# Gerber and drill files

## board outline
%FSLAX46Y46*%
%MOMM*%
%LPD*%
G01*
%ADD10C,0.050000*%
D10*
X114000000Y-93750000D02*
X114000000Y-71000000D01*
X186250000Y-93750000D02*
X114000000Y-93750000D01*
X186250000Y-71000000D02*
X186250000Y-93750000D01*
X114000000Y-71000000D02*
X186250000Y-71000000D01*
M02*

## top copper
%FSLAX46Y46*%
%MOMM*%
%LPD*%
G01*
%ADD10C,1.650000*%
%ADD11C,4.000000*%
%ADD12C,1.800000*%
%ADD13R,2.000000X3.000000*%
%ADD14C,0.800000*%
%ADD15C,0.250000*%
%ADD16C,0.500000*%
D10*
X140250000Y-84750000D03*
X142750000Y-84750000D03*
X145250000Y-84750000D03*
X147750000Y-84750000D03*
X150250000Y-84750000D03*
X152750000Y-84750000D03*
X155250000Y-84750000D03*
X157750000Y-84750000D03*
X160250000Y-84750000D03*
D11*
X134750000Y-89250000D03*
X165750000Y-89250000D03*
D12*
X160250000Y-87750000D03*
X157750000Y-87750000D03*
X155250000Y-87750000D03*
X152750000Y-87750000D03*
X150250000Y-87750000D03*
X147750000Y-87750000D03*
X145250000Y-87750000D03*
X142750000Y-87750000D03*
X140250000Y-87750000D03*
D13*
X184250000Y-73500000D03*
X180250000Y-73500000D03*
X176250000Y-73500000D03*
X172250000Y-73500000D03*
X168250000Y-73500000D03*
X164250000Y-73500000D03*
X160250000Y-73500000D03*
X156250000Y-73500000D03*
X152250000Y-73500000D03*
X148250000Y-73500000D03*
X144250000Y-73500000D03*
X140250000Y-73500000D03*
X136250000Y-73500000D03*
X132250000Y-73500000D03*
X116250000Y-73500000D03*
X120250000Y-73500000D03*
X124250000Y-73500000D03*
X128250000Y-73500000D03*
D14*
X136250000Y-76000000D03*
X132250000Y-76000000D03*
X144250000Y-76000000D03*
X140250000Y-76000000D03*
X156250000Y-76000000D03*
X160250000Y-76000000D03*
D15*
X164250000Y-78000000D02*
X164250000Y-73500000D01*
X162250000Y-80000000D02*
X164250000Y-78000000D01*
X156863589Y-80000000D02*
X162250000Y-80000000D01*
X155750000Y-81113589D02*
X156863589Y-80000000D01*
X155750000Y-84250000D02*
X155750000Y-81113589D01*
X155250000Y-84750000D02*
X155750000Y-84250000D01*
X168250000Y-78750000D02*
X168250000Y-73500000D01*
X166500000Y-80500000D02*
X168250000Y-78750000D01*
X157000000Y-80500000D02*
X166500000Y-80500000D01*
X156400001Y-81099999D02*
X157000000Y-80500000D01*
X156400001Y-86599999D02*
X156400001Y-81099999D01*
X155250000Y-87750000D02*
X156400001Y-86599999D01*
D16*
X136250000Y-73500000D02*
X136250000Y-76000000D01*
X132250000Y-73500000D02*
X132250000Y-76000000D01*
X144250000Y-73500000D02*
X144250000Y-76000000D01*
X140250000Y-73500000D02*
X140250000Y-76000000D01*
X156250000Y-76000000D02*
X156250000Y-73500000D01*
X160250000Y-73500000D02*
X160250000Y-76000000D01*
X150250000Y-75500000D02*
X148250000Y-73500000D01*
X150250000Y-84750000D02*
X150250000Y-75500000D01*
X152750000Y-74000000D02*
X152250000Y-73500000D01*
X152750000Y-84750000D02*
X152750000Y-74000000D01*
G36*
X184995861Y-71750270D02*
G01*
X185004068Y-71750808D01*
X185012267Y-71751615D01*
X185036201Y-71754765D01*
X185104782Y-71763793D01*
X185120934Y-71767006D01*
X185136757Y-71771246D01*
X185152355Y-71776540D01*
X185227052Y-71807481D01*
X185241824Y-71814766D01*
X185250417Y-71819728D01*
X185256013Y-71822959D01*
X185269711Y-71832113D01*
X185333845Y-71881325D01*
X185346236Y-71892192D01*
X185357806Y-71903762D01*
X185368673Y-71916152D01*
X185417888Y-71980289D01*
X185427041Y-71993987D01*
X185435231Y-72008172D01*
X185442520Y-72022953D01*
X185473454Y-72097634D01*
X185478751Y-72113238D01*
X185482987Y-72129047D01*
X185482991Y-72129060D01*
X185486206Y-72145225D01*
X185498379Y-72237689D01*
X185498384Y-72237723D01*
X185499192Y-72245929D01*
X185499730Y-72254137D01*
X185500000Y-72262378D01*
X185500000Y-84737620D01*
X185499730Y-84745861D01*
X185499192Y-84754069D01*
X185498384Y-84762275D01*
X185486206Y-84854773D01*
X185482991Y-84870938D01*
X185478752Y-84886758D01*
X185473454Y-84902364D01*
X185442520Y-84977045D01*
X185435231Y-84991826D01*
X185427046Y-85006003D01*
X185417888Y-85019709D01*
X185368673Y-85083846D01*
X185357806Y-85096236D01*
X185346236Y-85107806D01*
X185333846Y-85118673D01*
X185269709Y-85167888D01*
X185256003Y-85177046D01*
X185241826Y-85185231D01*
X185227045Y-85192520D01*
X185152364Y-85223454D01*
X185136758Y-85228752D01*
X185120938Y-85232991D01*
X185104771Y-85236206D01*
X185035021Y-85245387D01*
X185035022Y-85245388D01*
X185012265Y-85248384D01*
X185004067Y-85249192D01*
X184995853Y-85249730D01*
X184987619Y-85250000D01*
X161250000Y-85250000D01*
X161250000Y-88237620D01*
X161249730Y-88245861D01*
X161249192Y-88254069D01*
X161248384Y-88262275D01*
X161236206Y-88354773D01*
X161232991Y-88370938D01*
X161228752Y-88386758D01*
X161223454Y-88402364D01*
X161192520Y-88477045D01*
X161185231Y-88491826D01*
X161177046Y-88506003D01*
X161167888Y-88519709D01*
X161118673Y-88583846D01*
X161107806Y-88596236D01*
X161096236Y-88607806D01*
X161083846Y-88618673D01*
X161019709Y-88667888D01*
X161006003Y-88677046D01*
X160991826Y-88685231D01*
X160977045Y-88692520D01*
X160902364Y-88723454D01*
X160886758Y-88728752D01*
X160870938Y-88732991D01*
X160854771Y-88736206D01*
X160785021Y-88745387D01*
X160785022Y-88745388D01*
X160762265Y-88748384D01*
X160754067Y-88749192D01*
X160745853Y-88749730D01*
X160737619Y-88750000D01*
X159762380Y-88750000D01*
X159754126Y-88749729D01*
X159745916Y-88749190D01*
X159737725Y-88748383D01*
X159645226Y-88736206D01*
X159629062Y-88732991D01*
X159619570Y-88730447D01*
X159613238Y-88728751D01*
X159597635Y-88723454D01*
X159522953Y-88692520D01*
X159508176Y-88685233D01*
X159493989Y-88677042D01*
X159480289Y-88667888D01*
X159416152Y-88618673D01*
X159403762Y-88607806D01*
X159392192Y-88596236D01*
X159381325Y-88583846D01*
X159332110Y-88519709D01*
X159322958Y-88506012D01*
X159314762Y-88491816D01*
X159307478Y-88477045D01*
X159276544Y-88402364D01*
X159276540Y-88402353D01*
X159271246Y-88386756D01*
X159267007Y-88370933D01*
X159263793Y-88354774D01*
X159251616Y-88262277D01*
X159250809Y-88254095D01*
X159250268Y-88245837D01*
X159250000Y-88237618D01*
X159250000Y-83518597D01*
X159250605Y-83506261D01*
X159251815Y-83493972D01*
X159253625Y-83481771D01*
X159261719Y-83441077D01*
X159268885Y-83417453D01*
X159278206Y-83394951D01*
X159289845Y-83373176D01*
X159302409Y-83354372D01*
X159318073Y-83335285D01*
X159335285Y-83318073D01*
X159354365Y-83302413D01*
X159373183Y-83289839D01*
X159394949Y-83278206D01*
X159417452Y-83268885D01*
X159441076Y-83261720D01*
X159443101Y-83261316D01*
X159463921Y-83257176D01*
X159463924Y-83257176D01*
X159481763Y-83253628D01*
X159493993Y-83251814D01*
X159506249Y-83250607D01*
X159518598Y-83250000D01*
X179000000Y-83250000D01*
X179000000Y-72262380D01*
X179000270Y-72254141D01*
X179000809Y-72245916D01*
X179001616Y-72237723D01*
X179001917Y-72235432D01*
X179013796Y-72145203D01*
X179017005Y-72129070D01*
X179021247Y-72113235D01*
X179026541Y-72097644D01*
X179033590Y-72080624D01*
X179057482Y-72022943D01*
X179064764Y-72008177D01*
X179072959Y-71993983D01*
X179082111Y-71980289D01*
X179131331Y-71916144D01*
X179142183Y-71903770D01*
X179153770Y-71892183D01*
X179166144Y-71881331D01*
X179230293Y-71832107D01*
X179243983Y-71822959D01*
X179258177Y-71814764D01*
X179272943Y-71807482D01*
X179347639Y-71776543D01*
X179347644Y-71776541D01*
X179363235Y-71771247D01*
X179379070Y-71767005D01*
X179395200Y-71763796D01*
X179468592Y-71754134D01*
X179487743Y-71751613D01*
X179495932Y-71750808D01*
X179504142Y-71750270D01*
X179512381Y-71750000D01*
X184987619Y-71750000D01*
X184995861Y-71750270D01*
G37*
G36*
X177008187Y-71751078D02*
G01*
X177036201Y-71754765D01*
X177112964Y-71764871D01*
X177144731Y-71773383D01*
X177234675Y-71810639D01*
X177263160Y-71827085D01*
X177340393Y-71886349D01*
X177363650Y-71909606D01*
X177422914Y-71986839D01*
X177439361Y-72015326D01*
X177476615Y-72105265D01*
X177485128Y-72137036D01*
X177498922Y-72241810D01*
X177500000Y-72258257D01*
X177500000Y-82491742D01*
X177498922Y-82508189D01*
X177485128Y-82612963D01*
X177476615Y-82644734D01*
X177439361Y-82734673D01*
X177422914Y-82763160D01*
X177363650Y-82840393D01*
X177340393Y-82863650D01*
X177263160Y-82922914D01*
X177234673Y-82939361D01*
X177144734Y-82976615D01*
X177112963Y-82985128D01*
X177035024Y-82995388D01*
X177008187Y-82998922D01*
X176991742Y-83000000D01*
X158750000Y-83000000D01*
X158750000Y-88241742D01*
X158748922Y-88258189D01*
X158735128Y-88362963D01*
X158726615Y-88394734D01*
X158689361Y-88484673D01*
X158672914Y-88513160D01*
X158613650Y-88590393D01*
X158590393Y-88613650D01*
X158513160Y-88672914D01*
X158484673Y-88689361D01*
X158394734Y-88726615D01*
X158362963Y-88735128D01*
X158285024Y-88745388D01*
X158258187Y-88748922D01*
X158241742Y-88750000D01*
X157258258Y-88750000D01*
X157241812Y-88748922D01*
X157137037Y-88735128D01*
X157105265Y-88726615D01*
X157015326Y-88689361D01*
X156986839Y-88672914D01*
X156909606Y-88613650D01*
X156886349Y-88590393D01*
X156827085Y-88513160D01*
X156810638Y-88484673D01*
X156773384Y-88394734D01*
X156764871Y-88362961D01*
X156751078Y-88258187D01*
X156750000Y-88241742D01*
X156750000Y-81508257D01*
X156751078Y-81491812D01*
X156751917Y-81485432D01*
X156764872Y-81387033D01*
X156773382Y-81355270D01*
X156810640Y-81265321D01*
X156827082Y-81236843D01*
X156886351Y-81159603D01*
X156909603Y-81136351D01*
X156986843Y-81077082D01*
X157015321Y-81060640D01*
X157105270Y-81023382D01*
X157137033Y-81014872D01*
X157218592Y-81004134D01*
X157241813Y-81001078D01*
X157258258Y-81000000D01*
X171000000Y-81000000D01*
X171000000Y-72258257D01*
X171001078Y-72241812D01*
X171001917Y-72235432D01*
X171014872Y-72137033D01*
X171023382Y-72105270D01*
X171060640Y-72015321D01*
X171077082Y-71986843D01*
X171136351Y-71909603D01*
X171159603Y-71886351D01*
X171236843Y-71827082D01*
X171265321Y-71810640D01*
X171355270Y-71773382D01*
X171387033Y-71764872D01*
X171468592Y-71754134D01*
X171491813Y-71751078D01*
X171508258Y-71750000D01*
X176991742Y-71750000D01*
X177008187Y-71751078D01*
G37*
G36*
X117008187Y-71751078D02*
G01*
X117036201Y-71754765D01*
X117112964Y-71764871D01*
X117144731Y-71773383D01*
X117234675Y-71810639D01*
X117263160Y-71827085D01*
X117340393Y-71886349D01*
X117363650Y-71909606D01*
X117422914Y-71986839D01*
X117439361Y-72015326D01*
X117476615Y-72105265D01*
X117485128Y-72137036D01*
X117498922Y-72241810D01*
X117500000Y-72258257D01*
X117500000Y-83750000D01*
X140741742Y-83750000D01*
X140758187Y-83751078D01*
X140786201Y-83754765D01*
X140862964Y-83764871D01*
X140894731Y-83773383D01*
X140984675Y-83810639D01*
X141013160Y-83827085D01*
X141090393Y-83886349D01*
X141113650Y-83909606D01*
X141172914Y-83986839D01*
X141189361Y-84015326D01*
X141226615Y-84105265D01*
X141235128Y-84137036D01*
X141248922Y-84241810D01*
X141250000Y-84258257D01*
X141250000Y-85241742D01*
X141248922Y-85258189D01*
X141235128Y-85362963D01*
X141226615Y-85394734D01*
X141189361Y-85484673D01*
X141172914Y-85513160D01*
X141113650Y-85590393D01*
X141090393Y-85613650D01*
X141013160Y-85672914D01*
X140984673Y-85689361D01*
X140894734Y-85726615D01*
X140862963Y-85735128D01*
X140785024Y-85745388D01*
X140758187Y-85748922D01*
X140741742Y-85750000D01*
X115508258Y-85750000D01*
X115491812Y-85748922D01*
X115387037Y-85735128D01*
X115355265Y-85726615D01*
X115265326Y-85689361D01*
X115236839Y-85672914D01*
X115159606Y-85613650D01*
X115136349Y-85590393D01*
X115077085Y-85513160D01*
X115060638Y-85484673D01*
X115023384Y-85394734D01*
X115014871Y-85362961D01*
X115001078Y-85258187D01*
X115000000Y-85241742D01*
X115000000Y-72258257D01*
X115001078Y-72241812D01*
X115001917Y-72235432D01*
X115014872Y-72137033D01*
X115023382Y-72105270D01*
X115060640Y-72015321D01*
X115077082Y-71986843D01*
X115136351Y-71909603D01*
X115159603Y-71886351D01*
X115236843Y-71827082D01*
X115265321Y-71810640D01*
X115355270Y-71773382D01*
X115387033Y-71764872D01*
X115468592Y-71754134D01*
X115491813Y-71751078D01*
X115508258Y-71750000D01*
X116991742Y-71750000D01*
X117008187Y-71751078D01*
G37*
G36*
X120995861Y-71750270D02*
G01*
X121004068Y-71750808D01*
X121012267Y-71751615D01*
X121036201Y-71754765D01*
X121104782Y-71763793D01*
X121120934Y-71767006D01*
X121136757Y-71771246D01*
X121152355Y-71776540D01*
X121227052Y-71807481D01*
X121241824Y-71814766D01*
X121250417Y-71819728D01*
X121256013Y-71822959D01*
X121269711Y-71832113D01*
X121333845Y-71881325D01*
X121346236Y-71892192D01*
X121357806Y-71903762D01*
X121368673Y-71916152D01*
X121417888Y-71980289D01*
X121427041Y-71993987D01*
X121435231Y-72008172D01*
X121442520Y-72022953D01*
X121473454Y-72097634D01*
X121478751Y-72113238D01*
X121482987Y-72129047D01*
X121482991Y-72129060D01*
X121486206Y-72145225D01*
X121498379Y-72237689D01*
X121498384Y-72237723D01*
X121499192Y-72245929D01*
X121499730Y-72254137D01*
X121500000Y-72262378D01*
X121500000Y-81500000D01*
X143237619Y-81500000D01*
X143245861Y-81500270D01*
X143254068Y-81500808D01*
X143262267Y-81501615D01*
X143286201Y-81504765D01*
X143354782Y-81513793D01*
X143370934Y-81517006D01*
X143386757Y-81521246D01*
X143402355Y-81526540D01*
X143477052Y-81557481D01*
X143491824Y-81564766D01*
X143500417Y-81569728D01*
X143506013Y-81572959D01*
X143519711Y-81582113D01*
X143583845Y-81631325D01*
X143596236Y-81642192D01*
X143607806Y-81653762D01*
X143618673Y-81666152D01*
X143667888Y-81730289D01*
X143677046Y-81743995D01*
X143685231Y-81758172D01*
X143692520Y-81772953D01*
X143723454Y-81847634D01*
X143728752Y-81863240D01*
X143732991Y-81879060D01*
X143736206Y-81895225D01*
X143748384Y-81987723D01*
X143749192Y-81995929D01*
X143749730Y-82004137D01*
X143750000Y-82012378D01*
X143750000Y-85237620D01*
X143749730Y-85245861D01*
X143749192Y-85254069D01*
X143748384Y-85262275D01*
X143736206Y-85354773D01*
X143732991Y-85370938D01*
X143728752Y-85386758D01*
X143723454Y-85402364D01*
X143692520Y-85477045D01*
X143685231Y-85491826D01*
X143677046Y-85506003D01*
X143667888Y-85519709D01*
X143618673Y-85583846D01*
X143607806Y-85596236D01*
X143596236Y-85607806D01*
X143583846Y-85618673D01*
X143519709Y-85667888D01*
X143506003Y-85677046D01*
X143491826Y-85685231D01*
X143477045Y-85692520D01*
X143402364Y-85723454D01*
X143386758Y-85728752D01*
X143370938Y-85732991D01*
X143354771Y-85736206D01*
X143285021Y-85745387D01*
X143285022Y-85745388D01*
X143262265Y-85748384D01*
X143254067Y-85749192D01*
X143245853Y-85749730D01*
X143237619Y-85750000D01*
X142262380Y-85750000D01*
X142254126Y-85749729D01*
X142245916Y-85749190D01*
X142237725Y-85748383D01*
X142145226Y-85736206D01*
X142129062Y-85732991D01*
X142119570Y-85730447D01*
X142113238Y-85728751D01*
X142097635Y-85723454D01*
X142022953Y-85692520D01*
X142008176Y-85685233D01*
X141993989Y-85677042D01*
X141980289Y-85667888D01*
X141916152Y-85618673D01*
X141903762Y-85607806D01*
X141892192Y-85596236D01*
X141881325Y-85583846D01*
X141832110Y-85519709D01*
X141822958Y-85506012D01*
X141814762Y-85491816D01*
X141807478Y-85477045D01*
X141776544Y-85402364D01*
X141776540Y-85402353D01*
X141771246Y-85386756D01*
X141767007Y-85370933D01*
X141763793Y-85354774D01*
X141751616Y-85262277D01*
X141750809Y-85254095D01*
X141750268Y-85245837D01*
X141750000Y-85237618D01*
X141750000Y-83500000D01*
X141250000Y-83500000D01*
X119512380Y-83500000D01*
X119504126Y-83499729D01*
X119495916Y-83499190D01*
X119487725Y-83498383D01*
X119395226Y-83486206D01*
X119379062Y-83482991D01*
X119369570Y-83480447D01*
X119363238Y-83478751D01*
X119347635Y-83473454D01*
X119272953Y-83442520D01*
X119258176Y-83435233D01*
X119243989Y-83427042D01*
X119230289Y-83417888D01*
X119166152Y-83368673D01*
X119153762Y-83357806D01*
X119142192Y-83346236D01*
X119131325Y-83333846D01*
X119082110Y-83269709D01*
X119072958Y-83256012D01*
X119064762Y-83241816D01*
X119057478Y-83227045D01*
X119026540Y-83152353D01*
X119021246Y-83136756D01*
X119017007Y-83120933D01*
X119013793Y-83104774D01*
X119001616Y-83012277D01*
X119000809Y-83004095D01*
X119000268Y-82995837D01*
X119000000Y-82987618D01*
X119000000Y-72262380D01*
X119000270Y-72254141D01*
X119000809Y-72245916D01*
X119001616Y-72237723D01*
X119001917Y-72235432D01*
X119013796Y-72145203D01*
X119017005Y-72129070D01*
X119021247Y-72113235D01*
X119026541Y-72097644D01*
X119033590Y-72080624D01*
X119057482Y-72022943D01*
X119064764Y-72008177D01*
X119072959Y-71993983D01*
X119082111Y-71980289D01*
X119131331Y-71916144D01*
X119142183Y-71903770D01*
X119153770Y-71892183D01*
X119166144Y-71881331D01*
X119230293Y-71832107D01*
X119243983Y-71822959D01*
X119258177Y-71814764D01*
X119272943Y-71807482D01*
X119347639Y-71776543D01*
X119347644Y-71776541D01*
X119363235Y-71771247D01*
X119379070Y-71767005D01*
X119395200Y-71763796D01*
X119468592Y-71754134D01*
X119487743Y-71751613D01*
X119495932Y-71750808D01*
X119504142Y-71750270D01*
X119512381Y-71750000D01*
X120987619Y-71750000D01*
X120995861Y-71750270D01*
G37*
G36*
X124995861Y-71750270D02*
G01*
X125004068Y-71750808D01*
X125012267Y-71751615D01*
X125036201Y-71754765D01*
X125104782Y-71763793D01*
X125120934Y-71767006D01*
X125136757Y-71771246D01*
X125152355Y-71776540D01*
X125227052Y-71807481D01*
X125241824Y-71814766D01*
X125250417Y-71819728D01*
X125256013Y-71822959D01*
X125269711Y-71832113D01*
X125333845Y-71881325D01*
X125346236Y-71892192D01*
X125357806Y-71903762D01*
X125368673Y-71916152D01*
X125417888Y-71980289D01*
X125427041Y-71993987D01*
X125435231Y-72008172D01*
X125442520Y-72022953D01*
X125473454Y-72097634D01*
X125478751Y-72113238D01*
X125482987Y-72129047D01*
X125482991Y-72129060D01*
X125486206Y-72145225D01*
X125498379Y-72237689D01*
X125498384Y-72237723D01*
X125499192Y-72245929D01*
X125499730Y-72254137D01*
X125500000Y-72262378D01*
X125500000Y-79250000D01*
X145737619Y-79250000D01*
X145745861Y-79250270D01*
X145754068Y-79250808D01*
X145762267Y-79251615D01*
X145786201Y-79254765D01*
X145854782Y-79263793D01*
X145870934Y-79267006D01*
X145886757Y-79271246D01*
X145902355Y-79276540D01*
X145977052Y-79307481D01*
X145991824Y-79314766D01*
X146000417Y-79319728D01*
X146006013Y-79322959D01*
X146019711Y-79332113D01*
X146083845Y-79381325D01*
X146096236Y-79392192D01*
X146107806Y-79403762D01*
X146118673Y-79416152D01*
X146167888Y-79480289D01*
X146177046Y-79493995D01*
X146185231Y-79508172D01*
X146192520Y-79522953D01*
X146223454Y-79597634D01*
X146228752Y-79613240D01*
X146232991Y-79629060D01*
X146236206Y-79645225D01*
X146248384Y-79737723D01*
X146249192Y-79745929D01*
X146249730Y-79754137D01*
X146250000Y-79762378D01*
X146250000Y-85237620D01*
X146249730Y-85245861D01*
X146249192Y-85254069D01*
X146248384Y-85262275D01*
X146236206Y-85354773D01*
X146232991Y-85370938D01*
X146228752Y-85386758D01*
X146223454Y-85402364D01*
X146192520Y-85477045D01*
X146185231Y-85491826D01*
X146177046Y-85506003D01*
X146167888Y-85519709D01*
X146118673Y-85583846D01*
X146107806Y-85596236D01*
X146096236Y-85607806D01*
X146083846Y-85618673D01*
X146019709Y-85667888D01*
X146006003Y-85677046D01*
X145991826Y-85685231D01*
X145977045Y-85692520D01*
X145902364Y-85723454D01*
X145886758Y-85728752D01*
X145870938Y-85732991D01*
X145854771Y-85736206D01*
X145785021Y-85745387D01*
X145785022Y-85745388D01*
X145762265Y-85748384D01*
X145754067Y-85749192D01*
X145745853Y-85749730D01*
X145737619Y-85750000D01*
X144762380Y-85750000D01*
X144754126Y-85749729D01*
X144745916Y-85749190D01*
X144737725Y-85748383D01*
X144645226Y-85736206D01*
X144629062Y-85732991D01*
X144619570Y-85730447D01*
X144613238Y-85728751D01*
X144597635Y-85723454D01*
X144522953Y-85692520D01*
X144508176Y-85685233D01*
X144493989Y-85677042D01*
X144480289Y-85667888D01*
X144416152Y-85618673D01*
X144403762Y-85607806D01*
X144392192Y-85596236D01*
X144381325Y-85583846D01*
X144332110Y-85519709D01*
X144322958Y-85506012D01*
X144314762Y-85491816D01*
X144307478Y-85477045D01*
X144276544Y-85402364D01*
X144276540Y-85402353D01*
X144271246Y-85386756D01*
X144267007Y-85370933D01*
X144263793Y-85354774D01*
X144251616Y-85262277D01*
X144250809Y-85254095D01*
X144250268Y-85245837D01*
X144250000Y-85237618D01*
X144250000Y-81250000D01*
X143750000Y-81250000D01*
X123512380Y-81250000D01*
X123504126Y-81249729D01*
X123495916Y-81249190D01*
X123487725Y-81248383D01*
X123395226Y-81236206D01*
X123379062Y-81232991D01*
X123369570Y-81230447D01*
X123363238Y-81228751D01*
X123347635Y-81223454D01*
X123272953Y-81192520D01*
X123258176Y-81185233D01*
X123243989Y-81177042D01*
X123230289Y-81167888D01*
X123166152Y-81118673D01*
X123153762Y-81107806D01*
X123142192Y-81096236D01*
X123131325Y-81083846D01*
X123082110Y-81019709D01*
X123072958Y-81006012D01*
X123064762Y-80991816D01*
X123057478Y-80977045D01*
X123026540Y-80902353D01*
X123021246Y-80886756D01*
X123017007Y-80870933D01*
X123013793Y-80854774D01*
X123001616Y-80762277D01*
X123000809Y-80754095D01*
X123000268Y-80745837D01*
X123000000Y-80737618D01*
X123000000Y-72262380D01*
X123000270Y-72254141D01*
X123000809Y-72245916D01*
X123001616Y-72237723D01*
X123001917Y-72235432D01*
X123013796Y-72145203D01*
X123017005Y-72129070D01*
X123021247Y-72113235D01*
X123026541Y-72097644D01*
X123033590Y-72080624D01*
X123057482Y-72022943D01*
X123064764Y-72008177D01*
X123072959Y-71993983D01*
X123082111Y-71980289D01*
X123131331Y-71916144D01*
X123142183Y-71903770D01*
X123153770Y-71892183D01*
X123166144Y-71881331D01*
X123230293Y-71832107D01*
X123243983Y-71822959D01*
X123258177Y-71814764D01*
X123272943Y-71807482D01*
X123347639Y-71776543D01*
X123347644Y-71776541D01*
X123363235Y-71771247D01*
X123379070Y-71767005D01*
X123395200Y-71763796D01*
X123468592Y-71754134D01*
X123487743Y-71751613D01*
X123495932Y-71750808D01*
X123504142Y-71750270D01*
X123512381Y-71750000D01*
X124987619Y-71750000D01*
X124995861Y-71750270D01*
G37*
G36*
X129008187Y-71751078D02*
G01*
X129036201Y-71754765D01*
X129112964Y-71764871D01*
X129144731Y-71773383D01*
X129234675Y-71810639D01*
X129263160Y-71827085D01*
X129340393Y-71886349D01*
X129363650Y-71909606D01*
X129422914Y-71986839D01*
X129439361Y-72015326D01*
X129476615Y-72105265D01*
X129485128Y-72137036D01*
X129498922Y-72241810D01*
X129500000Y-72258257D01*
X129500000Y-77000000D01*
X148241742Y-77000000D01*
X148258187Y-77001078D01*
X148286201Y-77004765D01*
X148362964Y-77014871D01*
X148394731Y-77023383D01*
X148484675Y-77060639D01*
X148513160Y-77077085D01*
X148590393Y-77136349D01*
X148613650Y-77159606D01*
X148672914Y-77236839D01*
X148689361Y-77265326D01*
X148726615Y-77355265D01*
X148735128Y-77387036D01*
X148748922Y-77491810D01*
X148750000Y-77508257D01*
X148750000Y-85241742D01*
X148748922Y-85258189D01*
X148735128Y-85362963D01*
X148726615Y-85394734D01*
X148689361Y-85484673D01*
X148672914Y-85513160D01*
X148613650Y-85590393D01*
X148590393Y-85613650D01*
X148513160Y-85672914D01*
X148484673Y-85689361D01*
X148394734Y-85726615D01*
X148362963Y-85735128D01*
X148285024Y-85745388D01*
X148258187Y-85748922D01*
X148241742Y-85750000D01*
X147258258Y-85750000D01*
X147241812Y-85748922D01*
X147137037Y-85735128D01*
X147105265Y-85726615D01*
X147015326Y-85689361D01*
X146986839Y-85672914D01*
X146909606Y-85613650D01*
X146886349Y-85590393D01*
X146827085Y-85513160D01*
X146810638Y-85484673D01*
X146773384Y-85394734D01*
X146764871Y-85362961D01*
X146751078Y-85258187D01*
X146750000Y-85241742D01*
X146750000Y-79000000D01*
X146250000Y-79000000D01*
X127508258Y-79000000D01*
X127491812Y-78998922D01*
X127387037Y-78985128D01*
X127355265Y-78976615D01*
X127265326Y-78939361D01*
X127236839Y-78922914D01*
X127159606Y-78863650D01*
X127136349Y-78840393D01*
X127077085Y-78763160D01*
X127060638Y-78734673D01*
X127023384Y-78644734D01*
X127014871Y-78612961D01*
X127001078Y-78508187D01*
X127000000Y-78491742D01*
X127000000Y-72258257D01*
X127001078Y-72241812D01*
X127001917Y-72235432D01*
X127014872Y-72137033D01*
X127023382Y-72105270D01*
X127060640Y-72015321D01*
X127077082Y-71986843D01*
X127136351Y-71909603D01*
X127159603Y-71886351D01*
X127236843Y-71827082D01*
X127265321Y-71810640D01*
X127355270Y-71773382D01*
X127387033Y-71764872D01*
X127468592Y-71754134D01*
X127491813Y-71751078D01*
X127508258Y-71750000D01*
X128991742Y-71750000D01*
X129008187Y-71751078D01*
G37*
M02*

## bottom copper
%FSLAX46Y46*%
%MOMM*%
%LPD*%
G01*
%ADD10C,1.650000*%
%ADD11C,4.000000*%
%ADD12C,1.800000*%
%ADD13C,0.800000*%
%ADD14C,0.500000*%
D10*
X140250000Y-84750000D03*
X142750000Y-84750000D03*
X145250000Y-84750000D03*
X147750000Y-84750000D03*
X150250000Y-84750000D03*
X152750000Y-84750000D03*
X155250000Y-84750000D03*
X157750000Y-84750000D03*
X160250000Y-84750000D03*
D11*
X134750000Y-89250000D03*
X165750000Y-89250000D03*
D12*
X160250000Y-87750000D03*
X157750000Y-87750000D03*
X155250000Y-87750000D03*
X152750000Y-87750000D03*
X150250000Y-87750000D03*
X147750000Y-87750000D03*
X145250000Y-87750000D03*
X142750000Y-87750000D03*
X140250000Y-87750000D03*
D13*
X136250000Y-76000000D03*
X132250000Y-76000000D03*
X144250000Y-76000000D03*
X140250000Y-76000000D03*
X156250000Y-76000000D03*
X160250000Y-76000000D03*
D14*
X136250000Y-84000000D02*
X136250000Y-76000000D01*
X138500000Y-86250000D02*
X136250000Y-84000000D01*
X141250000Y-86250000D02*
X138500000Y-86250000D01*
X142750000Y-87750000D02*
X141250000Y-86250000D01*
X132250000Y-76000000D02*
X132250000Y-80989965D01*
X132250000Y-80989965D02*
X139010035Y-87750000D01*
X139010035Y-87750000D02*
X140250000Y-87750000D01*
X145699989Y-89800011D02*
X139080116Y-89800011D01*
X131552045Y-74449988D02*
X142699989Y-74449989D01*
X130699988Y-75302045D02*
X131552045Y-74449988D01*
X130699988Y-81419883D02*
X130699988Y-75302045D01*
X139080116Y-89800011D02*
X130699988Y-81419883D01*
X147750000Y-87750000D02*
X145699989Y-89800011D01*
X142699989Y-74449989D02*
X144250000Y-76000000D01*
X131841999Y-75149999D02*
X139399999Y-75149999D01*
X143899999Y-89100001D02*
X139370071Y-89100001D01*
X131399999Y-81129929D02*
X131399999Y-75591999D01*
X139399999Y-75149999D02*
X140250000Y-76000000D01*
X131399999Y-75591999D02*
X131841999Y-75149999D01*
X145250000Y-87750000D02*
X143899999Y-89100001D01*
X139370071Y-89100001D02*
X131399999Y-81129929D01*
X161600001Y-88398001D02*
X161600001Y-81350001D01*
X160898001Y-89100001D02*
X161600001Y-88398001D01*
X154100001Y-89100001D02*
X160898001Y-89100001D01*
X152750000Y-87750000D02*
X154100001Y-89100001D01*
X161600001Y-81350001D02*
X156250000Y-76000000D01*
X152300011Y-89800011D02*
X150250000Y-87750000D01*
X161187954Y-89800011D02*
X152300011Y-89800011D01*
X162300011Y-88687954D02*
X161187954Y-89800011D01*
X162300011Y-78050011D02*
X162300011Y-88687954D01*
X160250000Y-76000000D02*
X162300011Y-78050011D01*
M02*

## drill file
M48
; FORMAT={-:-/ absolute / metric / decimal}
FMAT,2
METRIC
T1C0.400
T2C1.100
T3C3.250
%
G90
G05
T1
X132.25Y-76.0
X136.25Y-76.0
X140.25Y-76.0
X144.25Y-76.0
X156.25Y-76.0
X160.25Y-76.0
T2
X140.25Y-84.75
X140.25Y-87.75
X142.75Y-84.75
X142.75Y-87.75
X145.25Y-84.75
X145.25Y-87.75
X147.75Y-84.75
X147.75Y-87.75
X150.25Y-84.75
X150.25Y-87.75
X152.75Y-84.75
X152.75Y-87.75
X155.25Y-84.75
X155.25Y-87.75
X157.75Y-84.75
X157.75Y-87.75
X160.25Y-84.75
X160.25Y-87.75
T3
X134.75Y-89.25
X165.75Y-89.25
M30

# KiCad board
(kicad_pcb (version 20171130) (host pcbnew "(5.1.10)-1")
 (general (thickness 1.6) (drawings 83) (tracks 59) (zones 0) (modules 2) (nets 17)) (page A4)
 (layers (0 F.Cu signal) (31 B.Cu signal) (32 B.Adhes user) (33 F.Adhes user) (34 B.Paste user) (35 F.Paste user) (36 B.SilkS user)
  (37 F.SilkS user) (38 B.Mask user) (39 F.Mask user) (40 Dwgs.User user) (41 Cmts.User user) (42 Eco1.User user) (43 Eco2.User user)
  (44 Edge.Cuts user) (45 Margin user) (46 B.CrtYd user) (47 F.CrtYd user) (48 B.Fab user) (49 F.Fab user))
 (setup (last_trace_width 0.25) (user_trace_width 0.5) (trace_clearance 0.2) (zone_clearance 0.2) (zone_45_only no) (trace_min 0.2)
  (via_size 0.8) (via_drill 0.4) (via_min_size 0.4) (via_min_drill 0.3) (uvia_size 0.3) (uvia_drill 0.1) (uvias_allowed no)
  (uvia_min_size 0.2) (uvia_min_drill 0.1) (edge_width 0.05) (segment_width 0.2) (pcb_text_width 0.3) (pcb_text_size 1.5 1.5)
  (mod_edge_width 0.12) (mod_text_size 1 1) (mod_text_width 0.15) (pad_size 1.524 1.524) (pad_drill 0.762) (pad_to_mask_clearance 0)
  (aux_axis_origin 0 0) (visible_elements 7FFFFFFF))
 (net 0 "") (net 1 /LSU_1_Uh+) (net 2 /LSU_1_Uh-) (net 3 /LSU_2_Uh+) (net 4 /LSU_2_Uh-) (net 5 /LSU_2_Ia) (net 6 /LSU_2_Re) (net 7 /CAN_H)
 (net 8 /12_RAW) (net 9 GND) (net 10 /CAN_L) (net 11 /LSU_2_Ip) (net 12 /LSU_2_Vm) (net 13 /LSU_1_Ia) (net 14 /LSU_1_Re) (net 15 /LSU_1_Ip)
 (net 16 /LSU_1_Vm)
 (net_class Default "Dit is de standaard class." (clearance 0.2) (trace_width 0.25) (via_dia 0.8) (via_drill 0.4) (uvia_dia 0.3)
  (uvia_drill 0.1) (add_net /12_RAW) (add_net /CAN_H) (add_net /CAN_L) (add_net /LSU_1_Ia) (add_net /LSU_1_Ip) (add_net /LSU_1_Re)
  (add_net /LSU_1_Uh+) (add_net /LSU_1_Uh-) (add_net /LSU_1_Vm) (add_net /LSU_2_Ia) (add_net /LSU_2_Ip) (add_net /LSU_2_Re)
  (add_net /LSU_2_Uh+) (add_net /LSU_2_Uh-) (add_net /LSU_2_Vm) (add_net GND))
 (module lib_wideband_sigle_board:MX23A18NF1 (layer F.Cu) (at 150.25 87.75)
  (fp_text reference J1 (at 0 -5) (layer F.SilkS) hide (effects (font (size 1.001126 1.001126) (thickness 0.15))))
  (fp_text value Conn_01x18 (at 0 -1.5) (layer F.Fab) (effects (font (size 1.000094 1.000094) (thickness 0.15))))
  (pad 18 thru_hole circle (at -10 -3) (size 1.65 1.65) (drill 1.1) (layers *.Cu *.Mask) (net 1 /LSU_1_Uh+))
  (pad 17 thru_hole circle (at -7.5 -3) (size 1.65 1.65) (drill 1.1) (layers *.Cu *.Mask) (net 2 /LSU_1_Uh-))
  (pad 16 thru_hole circle (at -5 -3) (size 1.65 1.65) (drill 1.1) (layers *.Cu *.Mask) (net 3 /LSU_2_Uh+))
  (pad 15 thru_hole circle (at -2.5 -3) (size 1.65 1.65) (drill 1.1) (layers *.Cu *.Mask) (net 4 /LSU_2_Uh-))
  (pad 14 thru_hole circle (at 0 -3) (size 1.65 1.65) (drill 1.1) (layers *.Cu *.Mask) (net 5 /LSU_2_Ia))
  (pad 13 thru_hole circle (at 2.5 -3) (size 1.65 1.65) (drill 1.1) (layers *.Cu *.Mask) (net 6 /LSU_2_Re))
  (pad 12 thru_hole circle (at 5 -3) (size 1.65 1.65) (drill 1.1) (layers *.Cu *.Mask) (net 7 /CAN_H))
  (pad 11 thru_hole circle (at 7.5 -3) (size 1.65 1.65) (drill 1.1) (layers *.Cu *.Mask) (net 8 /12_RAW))
  (pad 10 thru_hole circle (at 10 -3) (size 1.65 1.65) (drill 1.1) (layers *.Cu *.Mask) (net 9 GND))
  (pad "" thru_hole circle (at -15.5 1.5) (size 4 4) (drill 3.25) (layers *.Cu *.Mask))
  (pad "" thru_hole circle (at 15.5 1.5) (size 4 4) (drill 3.25) (layers *.Cu *.Mask))
  (pad 9 thru_hole circle (at 10 0) (size 1.8 1.8) (drill 1.1) (layers *.Cu *.Mask) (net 9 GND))
  (pad 8 thru_hole circle (at 7.5 0) (size 1.8 1.8) (drill 1.1) (layers *.Cu *.Mask) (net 8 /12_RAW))
  (pad 7 thru_hole circle (at 5 0) (size 1.8 1.8) (drill 1.1) (layers *.Cu *.Mask) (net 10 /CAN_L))
  (pad 6 thru_hole circle (at 2.5 0) (size 1.8 1.8) (drill 1.1) (layers *.Cu *.Mask) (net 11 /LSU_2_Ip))
  (pad 5 thru_hole circle (at 0 0) (size 1.8 1.8) (drill 1.1) (layers *.Cu *.Mask) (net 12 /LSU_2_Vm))
  (pad 4 thru_hole circle (at -2.5 0) (size 1.8 1.8) (drill 1.1) (layers *.Cu *.Mask) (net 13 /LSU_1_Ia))
  (pad 3 thru_hole circle (at -5 0) (size 1.8 1.8) (drill 1.1) (layers *.Cu *.Mask) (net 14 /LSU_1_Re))
  (pad 2 thru_hole circle (at -7.5 0) (size 1.8 1.8) (drill 1.1) (layers *.Cu *.Mask) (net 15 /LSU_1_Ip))
  (pad 1 thru_hole circle (at -10 0) (size 1.8 1.8) (drill 1.1) (layers *.Cu *.Mask) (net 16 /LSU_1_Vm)))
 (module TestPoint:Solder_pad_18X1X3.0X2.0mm (layer F.Cu) (at 150.25 73.5 180)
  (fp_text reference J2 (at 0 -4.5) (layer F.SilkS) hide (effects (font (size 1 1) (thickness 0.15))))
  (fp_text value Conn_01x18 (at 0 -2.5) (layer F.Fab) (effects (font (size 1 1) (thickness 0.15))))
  (pad 18 smd rect (at -34 0 180) (size 2 3) (layers F.Cu F.Paste F.Mask) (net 9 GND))
  (pad 17 smd rect (at -30 0 180) (size 2 3) (layers F.Cu F.Paste F.Mask) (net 9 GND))
  (pad 16 smd rect (at -26 0 180) (size 2 3) (layers F.Cu F.Paste F.Mask) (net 8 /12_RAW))
  (pad 15 smd rect (at -22 0 180) (size 2 3) (layers F.Cu F.Paste F.Mask) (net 8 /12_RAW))
  (pad 14 smd rect (at -18 0 180) (size 2 3) (layers F.Cu F.Paste F.Mask) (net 10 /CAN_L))
  (pad 13 smd rect (at -14 0 180) (size 2 3) (layers F.Cu F.Paste F.Mask) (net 7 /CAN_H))
  (pad 12 smd rect (at -10 0 180) (size 2 3) (layers F.Cu F.Paste F.Mask) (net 12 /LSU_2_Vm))
  (pad 11 smd rect (at -6 0 180) (size 2 3) (layers F.Cu F.Paste F.Mask) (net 11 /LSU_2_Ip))
  (pad 10 smd rect (at -2 0 180) (size 2 3) (layers F.Cu F.Paste F.Mask) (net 6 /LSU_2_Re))
  (pad 9 smd rect (at 2 0 180) (size 2 3) (layers F.Cu F.Paste F.Mask) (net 5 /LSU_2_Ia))
  (pad 8 smd rect (at 6 0 180) (size 2 3) (layers F.Cu F.Paste F.Mask) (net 13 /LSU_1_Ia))
  (pad 7 smd rect (at 10 0 180) (size 2 3) (layers F.Cu F.Paste F.Mask) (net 14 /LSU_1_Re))
  (pad 6 smd rect (at 14 0 180) (size 2 3) (layers F.Cu F.Paste F.Mask) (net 15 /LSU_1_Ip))
  (pad 5 smd rect (at 18 0 180) (size 2 3) (layers F.Cu F.Paste F.Mask) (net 16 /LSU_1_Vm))
  (pad 1 smd rect (at 34 0 180) (size 2 3) (layers F.Cu F.Paste F.Mask) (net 1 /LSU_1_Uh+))
  (pad 2 smd rect (at 30 0 180) (size 2 3) (layers F.Cu F.Paste F.Mask) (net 2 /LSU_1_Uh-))
  (pad 3 smd rect (at 26 0 180) (size 2 3) (layers F.Cu F.Paste F.Mask) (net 3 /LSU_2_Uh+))
  (pad 4 smd rect (at 22 0 180) (size 2 3) (layers F.Cu F.Paste F.Mask) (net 4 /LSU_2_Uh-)))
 (gr_line (start 114 93.75) (end 114 71) (layer Edge.Cuts) (width 0.05))
 (gr_line (start 186.25 93.75) (end 114 93.75) (layer Edge.Cuts) (width 0.05))
 (gr_line (start 186.25 71) (end 186.25 93.75) (layer Edge.Cuts) (width 0.05))
 (gr_line (start 114 71) (end 186.25 71) (layer Edge.Cuts) (width 0.05))
 (segment (start 164.25 78) (end 164.25 73.5) (width 0.25) (layer F.Cu) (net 7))
 (segment (start 162.25 80) (end 164.25 78) (width 0.25) (layer F.Cu) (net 7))
 (segment (start 156.863589 80) (end 162.25 80) (width 0.25) (layer F.Cu) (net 7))
 (segment (start 155.75 81.113589) (end 156.863589 80) (width 0.25) (layer F.Cu) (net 7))
 (segment (start 155.75 84.25) (end 155.75 81.113589) (width 0.25) (layer F.Cu) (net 7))
 (segment (start 155.25 84.75) (end 155.75 84.25) (width 0.25) (layer F.Cu) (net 7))
 (segment (start 168.25 78.75) (end 168.25 73.5) (width 0.25) (layer F.Cu) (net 10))
 (segment (start 166.5 80.5) (end 168.25 78.75) (width 0.25) (layer F.Cu) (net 10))
 (segment (start 157 80.5) (end 166.5 80.5) (width 0.25) (layer F.Cu) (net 10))
 (segment (start 156.400001 81.099999) (end 157 80.5) (width 0.25) (layer F.Cu) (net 10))
 (segment (start 156.400001 86.599999) (end 156.400001 81.099999) (width 0.25) (layer F.Cu) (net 10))
 (segment (start 155.25 87.75) (end 156.400001 86.599999) (width 0.25) (layer F.Cu) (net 10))
 (via (at 136.25 76) (size 0.8) (drill 0.4) (layers F.Cu B.Cu) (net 15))
 (segment (start 136.25 73.5) (end 136.25 76) (width 0.5) (layer F.Cu) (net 15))
 (segment (start 136.25 84) (end 136.25 76) (width 0.5) (layer B.Cu) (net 15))
 (segment (start 138.5 86.25) (end 136.25 84) (width 0.5) (layer B.Cu) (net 15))
 (segment (start 141.25 86.25) (end 138.5 86.25) (width 0.5) (layer B.Cu) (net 15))
 (segment (start 142.75 87.75) (end 141.25 86.25) (width 0.5) (layer B.Cu) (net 15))
 (via (at 132.25 76) (size 0.8) (drill 0.4) (layers F.Cu B.Cu) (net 16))
 (segment (start 132.25 73.5) (end 132.25 76) (width 0.5) (layer F.Cu) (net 16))
 (segment (start 132.25 76) (end 132.25 80.989965) (width 0.5) (layer B.Cu) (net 16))
 (segment (start 132.25 80.989965) (end 139.010035 87.75) (width 0.5) (layer B.Cu) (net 16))
 (segment (start 139.010035 87.75) (end 140.25 87.75) (width 0.5) (layer B.Cu) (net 16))
 (segment (start 144.25 73.5) (end 144.25 76) (width 0.5) (layer F.Cu) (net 13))
 (via (at 144.25 76) (size 0.8) (drill 0.4) (layers F.Cu B.Cu) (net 13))
 (segment (start 145.699989 89.800011) (end 139.080116 89.800011) (width 0.5) (layer B.Cu) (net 13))
 (segment (start 131.552045 74.449988) (end 142.699989 74.449989) (width 0.5) (layer B.Cu) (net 13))
 (segment (start 130.699988 75.302045) (end 131.552045 74.449988) (width 0.5) (layer B.Cu) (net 13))
 (segment (start 130.699988 81.419883) (end 130.699988 75.302045) (width 0.5) (layer B.Cu) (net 13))
 (segment (start 139.080116 89.800011) (end 130.699988 81.419883) (width 0.5) (layer B.Cu) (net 13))
 (segment (start 147.75 87.75) (end 145.699989 89.800011) (width 0.5) (layer B.Cu) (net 13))
 (segment (start 142.699989 74.449989) (end 144.25 76) (width 0.5) (layer B.Cu) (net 13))
 (via (at 140.25 76) (size 0.8) (drill 0.4) (layers F.Cu B.Cu) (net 14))
 (segment (start 140.25 73.5) (end 140.25 76) (width 0.5) (layer F.Cu) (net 14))
 (segment (start 131.841999 75.149999) (end 139.399999 75.149999) (width 0.5) (layer B.Cu) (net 14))
 (segment (start 143.899999 89.100001) (end 139.370071 89.100001) (width 0.5) (layer B.Cu) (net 14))
 (segment (start 131.399999 81.129929) (end 131.399999 75.591999) (width 0.5) (layer B.Cu) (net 14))
 (segment (start 139.399999 75.149999) (end 140.25 76) (width 0.5) (layer B.Cu) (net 14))
 (segment (start 131.399999 75.591999) (end 131.841999 75.149999) (width 0.5) (layer B.Cu) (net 14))
 (segment (start 145.25 87.75) (end 143.899999 89.100001) (width 0.5) (layer B.Cu) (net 14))
 (segment (start 139.370071 89.100001) (end 131.399999 81.129929) (width 0.5) (layer B.Cu) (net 14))
 (segment (start 161.600001 88.398001) (end 161.600001 81.350001) (width 0.5) (layer B.Cu) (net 11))
 (segment (start 160.898001 89.100001) (end 161.600001 88.398001) (width 0.5) (layer B.Cu) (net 11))
 (segment (start 154.100001 89.100001) (end 160.898001 89.100001) (width 0.5) (layer B.Cu) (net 11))
 (segment (start 152.75 87.75) (end 154.100001 89.100001) (width 0.5) (layer B.Cu) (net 11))
 (via (at 156.25 76) (size 0.8) (drill 0.4) (layers F.Cu B.Cu) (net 11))
 (segment (start 161.600001 81.350001) (end 156.25 76) (width 0.5) (layer B.Cu) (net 11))
 (segment (start 156.25 76) (end 156.25 73.5) (width 0.5) (layer F.Cu) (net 11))
 (via (at 160.25 76) (size 0.8) (drill 0.4) (layers F.Cu B.Cu) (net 12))
 (segment (start 160.25 73.5) (end 160.25 76) (width 0.5) (layer F.Cu) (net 12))
 (segment (start 152.300011 89.800011) (end 150.25 87.75) (width 0.5) (layer B.Cu) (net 12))
 (segment (start 161.187954 89.800011) (end 152.300011 89.800011) (width 0.5) (layer B.Cu) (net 12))
 (segment (start 162.300011 88.687954) (end 161.187954 89.800011) (width 0.5) (layer B.Cu) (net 12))
 (segment (start 162.300011 78.050011) (end 162.300011 88.687954) (width 0.5) (layer B.Cu) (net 12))
 (segment (start 160.25 76) (end 162.300011 78.050011) (width 0.5) (layer B.Cu) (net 12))
 (segment (start 150.25 75.5) (end 148.25 73.5) (width 0.5) (layer F.Cu) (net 5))
 (segment (start 150.25 84.75) (end 150.25 75.5) (width 0.5) (layer F.Cu) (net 5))
 (segment (start 152.75 74) (end 152.25 73.5) (width 0.5) (layer F.Cu) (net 6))
 (segment (start 152.75 84.75) (end 152.75 74) (width 0.5) (layer F.Cu) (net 6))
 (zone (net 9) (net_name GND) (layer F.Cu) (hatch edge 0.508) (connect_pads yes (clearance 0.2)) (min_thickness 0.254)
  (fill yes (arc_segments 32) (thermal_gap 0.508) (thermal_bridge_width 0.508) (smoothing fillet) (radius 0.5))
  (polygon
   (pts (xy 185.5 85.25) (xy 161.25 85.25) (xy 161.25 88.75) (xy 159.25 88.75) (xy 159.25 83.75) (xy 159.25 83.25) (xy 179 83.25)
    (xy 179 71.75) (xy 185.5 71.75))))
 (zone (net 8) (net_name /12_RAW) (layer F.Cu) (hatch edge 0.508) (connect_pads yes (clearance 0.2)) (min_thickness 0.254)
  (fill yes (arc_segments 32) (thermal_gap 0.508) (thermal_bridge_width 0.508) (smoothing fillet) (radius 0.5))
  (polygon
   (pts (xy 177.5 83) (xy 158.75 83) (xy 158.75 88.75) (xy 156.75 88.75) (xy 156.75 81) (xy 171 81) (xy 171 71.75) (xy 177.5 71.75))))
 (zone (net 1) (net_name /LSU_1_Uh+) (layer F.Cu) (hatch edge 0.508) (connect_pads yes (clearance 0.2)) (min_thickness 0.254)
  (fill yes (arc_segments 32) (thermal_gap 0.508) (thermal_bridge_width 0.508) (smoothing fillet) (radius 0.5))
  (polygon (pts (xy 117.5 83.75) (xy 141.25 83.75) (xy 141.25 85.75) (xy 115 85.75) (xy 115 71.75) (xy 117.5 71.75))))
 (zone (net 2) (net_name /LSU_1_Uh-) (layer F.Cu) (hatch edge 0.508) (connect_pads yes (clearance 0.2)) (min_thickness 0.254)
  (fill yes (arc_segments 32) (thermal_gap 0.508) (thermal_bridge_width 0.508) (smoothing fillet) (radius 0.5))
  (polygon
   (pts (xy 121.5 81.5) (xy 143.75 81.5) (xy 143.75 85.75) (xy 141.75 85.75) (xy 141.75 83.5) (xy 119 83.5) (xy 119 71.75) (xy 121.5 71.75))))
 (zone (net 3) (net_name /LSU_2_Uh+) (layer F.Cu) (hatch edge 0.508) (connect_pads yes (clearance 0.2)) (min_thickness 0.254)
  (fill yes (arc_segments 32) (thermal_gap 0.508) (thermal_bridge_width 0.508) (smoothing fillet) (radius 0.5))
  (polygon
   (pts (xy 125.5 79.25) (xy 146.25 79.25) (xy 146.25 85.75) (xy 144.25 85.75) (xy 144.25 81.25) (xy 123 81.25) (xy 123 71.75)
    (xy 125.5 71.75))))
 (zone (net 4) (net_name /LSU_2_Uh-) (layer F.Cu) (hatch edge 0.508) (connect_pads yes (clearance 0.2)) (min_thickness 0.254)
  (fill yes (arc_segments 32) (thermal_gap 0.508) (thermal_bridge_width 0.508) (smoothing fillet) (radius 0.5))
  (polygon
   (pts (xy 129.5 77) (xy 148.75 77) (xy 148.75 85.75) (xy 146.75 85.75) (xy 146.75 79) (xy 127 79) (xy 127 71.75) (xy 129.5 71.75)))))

